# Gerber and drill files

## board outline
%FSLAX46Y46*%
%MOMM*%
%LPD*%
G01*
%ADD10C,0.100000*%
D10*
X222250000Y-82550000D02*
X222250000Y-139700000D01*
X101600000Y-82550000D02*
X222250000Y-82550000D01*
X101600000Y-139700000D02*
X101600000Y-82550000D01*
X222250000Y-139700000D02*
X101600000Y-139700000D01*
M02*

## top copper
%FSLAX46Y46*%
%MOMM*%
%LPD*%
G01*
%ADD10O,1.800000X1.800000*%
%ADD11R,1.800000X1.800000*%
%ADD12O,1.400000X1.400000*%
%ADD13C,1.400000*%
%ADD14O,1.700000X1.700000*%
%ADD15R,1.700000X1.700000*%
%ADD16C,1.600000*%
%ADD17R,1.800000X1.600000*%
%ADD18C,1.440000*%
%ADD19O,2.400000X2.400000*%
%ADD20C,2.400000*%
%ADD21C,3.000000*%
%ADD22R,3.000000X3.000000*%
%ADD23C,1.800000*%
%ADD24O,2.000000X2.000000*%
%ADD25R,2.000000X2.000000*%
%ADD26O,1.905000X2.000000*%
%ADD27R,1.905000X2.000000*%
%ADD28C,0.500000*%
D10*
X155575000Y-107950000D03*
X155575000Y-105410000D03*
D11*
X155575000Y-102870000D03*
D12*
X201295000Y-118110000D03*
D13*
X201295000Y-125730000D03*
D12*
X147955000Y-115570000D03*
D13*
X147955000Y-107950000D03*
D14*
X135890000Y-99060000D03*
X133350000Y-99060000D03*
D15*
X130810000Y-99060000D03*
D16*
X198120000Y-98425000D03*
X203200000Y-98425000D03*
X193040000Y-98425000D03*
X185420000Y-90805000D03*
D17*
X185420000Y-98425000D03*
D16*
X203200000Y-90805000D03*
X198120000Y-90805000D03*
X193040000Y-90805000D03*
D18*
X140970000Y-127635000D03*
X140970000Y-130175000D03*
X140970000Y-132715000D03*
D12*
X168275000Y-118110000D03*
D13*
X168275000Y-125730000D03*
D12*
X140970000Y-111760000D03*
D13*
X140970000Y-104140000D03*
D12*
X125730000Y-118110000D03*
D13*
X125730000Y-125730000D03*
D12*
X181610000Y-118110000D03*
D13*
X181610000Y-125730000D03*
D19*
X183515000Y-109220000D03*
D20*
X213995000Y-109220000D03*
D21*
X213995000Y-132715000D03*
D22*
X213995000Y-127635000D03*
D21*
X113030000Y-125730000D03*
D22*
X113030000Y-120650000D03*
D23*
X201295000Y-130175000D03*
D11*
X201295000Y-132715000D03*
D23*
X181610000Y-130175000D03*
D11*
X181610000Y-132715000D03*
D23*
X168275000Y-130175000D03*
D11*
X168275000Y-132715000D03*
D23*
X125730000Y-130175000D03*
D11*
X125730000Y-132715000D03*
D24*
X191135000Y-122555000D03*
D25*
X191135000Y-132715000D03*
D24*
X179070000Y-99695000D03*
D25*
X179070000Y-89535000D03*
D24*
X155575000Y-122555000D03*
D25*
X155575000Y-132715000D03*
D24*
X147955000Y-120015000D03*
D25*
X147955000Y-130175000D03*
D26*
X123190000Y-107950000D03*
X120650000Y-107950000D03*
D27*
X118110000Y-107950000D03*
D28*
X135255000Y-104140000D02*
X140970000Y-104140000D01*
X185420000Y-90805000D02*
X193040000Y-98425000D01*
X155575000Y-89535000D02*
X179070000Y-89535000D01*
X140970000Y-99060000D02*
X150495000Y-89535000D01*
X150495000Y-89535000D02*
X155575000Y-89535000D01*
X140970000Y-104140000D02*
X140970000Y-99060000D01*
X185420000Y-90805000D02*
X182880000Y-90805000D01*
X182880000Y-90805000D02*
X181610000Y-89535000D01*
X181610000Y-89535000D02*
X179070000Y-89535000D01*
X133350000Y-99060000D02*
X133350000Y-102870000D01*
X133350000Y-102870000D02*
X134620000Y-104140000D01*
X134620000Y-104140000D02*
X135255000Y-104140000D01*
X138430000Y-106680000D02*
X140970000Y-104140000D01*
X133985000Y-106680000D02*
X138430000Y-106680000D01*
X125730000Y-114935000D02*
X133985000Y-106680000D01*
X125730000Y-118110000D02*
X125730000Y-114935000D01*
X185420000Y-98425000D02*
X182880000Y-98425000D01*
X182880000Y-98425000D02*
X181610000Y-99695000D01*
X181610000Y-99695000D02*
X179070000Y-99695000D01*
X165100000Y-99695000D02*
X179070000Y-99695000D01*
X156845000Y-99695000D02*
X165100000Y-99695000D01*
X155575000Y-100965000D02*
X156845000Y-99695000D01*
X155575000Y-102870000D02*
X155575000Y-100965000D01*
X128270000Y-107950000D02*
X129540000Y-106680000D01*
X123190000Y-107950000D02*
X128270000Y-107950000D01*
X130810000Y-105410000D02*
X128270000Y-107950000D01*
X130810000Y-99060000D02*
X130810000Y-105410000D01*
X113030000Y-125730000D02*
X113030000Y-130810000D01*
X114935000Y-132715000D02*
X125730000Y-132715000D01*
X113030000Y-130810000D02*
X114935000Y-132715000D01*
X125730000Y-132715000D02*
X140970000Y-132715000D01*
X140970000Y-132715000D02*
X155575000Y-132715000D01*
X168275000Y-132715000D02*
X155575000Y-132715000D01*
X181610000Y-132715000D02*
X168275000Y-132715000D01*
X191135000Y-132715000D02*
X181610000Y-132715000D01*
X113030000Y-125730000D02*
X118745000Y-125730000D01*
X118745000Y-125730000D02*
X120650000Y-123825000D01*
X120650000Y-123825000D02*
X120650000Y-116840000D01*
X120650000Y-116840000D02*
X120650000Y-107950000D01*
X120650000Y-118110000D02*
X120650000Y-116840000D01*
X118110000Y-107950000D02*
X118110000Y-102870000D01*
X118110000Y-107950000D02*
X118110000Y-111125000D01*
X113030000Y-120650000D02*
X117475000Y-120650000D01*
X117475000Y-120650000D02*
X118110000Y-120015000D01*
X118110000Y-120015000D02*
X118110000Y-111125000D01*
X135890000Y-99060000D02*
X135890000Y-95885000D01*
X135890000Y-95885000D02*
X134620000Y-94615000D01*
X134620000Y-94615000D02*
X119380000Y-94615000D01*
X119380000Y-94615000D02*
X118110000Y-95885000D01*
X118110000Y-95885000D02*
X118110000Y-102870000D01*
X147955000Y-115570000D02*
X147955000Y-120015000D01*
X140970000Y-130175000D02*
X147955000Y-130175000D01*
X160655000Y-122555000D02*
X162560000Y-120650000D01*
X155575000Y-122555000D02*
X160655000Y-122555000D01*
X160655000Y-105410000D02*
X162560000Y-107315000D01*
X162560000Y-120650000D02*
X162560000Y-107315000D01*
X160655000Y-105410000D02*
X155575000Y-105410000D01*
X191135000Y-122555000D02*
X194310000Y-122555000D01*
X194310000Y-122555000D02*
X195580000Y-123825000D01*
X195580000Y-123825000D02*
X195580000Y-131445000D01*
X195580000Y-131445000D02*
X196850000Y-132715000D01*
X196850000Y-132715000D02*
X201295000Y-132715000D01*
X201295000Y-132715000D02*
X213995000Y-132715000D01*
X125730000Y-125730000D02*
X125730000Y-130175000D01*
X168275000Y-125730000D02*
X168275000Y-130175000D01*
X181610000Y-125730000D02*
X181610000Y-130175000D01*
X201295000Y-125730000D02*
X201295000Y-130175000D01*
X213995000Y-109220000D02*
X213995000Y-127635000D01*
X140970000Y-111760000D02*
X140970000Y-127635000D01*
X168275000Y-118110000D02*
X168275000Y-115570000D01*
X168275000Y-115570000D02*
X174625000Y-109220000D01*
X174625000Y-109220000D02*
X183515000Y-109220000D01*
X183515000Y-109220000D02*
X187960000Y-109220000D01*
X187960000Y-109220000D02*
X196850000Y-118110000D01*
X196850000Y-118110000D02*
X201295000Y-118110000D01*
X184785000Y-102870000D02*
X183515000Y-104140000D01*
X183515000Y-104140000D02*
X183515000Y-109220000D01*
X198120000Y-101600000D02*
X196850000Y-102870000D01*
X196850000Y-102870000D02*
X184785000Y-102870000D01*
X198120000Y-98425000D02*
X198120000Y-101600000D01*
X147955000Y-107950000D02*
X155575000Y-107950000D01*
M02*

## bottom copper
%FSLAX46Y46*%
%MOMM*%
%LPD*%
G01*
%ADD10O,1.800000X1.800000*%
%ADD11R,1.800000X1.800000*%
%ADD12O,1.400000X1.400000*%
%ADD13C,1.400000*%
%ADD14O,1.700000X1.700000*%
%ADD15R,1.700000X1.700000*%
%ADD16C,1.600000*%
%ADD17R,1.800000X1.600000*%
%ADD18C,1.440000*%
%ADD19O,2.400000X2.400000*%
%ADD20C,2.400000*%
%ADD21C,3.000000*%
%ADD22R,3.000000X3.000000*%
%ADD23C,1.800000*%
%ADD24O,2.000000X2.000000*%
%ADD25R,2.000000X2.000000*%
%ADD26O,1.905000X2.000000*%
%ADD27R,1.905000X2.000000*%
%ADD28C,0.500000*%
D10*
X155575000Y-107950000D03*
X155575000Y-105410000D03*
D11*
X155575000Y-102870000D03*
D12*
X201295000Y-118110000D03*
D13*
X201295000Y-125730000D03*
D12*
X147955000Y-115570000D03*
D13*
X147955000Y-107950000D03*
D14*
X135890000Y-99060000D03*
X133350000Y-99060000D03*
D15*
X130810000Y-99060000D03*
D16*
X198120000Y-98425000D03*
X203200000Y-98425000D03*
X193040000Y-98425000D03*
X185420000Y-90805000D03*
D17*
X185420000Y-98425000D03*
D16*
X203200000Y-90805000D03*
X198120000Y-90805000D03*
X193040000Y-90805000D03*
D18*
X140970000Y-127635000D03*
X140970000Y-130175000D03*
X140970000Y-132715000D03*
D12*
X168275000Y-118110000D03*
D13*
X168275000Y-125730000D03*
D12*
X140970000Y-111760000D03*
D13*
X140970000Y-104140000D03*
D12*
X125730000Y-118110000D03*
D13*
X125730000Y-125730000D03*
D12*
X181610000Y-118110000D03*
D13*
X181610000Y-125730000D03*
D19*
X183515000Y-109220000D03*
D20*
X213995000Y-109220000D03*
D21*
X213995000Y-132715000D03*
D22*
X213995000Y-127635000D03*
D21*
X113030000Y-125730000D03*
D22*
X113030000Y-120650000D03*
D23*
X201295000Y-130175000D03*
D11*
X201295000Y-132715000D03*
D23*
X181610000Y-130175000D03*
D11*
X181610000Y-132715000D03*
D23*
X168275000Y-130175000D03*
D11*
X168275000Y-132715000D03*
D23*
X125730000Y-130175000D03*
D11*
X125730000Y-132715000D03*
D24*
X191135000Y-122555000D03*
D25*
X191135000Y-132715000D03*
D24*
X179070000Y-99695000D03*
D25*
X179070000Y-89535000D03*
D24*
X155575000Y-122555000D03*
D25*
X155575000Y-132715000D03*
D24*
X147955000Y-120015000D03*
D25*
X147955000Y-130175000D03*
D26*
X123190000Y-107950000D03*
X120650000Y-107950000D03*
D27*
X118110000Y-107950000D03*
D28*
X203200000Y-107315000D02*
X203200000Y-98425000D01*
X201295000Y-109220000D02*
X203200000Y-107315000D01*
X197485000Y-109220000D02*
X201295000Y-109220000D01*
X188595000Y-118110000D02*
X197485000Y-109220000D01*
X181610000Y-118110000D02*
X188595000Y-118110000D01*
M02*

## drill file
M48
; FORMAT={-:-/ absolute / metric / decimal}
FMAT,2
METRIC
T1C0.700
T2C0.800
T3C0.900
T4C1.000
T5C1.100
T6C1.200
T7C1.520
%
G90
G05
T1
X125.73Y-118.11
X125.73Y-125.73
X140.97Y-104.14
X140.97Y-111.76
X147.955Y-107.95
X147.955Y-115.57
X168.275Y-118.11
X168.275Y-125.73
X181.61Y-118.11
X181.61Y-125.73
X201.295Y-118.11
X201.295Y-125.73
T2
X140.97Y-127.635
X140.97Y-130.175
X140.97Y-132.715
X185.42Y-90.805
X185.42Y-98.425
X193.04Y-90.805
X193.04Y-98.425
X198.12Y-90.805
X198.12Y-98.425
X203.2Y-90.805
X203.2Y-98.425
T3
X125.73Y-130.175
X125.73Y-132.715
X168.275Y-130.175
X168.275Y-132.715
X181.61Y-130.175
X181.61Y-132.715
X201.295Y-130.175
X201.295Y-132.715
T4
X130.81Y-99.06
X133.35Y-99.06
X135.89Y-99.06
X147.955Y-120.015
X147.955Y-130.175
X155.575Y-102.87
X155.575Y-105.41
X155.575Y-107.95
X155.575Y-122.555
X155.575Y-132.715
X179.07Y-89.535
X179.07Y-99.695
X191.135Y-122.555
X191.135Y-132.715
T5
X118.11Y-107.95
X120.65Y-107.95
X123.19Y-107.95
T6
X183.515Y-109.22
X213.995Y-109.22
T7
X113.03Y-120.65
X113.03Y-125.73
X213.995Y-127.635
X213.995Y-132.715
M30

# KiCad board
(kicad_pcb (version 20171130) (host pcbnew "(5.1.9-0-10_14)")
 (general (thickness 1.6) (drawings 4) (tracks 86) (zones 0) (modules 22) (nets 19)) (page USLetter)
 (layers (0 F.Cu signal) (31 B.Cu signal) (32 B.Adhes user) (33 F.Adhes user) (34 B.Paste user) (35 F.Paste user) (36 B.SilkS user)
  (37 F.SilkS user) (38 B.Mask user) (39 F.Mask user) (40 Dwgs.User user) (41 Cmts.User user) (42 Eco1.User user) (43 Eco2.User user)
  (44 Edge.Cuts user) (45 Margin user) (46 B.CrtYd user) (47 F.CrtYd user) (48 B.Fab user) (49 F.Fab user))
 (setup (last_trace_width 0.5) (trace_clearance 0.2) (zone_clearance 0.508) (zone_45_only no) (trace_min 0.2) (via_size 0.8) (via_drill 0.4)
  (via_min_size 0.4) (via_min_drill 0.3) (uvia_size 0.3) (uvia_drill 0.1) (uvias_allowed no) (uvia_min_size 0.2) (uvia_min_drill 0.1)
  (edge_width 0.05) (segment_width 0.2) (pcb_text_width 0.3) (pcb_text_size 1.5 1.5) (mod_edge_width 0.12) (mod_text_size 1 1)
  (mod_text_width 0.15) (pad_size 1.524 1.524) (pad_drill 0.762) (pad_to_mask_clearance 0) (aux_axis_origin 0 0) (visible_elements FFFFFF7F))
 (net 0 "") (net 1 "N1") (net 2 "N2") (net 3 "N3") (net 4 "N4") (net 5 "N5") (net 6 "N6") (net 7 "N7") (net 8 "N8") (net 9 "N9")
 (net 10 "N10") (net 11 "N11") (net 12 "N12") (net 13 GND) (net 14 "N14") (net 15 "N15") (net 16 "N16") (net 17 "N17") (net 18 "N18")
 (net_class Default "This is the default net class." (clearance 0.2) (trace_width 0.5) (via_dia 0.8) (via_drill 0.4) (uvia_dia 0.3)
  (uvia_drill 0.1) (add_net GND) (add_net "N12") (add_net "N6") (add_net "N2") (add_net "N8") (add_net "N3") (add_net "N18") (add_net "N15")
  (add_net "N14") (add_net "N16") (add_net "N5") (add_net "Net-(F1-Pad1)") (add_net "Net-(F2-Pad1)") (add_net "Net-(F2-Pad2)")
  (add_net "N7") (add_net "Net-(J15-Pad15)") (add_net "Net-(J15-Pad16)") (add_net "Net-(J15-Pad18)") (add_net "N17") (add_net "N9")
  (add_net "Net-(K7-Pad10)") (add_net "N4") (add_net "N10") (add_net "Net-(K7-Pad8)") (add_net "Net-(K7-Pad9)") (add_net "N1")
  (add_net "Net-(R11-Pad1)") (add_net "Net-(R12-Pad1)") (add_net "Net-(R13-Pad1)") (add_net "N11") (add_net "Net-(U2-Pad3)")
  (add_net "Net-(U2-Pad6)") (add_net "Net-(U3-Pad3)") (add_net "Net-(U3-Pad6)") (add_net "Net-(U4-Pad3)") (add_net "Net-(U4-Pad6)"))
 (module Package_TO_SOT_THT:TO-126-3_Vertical (layer F.Cu) (at 155.575 102.87 270)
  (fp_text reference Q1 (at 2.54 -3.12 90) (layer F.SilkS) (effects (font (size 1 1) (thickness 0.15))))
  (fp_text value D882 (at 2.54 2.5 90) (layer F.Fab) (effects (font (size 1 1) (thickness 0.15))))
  (pad 3 thru_hole oval (at 5.08 0 270) (size 1.8 1.8) (drill 1) (layers *.Cu *.Mask) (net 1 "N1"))
  (pad 2 thru_hole oval (at 2.54 0 270) (size 1.8 1.8) (drill 1) (layers *.Cu *.Mask) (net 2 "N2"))
  (pad 1 thru_hole rect (at 0 0 270) (size 1.8 1.8) (drill 1) (layers *.Cu *.Mask) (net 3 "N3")))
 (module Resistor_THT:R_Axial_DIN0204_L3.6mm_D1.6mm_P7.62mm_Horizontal (layer F.Cu) (at 201.295 125.73 90)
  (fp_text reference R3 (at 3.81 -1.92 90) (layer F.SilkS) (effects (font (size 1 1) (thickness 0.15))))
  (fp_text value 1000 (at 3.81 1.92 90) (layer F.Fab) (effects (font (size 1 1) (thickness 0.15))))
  (pad 2 thru_hole oval (at 7.62 0 90) (size 1.4 1.4) (drill 0.7) (layers *.Cu *.Mask) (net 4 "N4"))
  (pad 1 thru_hole circle (at 0 0 90) (size 1.4 1.4) (drill 0.7) (layers *.Cu *.Mask) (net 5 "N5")))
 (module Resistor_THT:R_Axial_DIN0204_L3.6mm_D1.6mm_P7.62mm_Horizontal (layer F.Cu) (at 147.955 107.95 270)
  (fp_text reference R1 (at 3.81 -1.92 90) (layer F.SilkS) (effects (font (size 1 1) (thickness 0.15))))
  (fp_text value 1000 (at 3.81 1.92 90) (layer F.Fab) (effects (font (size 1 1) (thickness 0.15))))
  (pad 2 thru_hole oval (at 7.62 0 270) (size 1.4 1.4) (drill 0.7) (layers *.Cu *.Mask) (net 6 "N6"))
  (pad 1 thru_hole circle (at 0 0 270) (size 1.4 1.4) (drill 0.7) (layers *.Cu *.Mask) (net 1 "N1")))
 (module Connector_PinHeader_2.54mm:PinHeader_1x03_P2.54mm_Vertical (layer F.Cu) (at 130.81 99.06 90)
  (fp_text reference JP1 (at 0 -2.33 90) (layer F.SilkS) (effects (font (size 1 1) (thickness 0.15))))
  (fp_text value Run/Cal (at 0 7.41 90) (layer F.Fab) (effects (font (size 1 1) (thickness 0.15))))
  (pad 3 thru_hole oval (at 0 5.08 90) (size 1.7 1.7) (drill 1) (layers *.Cu *.Mask) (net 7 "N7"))
  (pad 2 thru_hole oval (at 0 2.54 90) (size 1.7 1.7) (drill 1) (layers *.Cu *.Mask) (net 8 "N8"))
  (pad 1 thru_hole rect (at 0 0 90) (size 1.7 1.7) (drill 1) (layers *.Cu *.Mask) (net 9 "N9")))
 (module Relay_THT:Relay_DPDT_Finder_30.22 (layer F.Cu) (at 185.42 98.425)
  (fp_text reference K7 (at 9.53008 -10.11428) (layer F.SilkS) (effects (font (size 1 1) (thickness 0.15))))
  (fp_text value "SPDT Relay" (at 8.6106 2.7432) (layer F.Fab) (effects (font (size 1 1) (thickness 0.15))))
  (pad 3 thru_hole circle (at 12.7 0 90) (size 1.6 1.6) (drill 0.8) (layers *.Cu *.Mask) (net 4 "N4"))
  (pad 5 thru_hole circle (at 17.78 0 90) (size 1.6 1.6) (drill 0.8) (layers *.Cu *.Mask) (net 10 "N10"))
  (pad 4 thru_hole circle (at 7.62 0 90) (size 1.6 1.6) (drill 0.8) (layers *.Cu *.Mask) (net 8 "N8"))
  (pad 12 thru_hole circle (at 0 -7.62 90) (size 1.6 1.6) (drill 0.8) (layers *.Cu *.Mask) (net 8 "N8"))
  (pad 1 thru_hole rect (at 0 0 90) (size 1.6 1.8) (drill 0.8) (layers *.Cu *.Mask) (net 3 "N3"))
  (pad 8 thru_hole circle (at 17.78 -7.62 180) (size 1.6 1.6) (drill 0.8) (layers *.Cu *.Mask))
  (pad 10 thru_hole circle (at 12.7 -7.62 90) (size 1.6 1.6) (drill 0.8) (layers *.Cu *.Mask))
  (pad 9 thru_hole circle (at 7.62 -7.62 90) (size 1.6 1.6) (drill 0.8) (layers *.Cu *.Mask)))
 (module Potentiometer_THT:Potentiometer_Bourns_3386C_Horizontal (layer F.Cu) (at 140.97 127.635)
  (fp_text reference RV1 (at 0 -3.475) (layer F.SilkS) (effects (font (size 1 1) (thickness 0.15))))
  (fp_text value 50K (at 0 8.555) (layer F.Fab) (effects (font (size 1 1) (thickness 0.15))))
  (pad 1 thru_hole circle (at 0 0) (size 1.44 1.44) (drill 0.8) (layers *.Cu *.Mask) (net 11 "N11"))
  (pad 2 thru_hole circle (at 0 2.54) (size 1.44 1.44) (drill 0.8) (layers *.Cu *.Mask) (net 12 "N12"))
  (pad 3 thru_hole circle (at 0 5.08) (size 1.44 1.44) (drill 0.8) (layers *.Cu *.Mask) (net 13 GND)))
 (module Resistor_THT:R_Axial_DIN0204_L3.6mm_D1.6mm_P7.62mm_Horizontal (layer F.Cu) (at 168.275 125.73 90)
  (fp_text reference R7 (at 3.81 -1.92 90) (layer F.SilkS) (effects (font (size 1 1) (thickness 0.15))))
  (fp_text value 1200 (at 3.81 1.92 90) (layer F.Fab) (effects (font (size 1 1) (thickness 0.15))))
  (pad 2 thru_hole oval (at 7.62 0 90) (size 1.4 1.4) (drill 0.7) (layers *.Cu *.Mask) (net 4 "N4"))
  (pad 1 thru_hole circle (at 0 0 90) (size 1.4 1.4) (drill 0.7) (layers *.Cu *.Mask) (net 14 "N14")))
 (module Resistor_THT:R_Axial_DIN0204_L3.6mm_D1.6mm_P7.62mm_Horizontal (layer F.Cu) (at 140.97 104.14 270)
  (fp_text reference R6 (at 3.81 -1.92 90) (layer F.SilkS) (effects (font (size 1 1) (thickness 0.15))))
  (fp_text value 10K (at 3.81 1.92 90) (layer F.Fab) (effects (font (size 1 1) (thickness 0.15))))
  (pad 2 thru_hole oval (at 7.62 0 270) (size 1.4 1.4) (drill 0.7) (layers *.Cu *.Mask) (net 11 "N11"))
  (pad 1 thru_hole circle (at 0 0 270) (size 1.4 1.4) (drill 0.7) (layers *.Cu *.Mask) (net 8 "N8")))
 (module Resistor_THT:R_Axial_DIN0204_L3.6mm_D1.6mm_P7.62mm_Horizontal (layer F.Cu) (at 125.73 125.73 90)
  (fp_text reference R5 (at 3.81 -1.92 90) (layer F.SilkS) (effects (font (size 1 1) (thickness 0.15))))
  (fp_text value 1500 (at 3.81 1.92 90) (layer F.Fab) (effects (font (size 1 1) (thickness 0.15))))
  (pad 2 thru_hole oval (at 7.62 0 90) (size 1.4 1.4) (drill 0.7) (layers *.Cu *.Mask) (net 8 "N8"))
  (pad 1 thru_hole circle (at 0 0 90) (size 1.4 1.4) (drill 0.7) (layers *.Cu *.Mask) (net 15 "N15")))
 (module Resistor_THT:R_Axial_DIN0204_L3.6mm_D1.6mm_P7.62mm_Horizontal (layer F.Cu) (at 181.61 125.73 90)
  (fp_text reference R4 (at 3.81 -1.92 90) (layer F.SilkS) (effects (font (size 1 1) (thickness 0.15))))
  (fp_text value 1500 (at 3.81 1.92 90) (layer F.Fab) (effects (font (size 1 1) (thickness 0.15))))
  (pad 2 thru_hole oval (at 7.62 0 90) (size 1.4 1.4) (drill 0.7) (layers *.Cu *.Mask) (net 10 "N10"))
  (pad 1 thru_hole circle (at 0 0 90) (size 1.4 1.4) (drill 0.7) (layers *.Cu *.Mask) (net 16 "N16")))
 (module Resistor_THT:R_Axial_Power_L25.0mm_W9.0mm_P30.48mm (layer F.Cu) (at 213.995 109.22 180)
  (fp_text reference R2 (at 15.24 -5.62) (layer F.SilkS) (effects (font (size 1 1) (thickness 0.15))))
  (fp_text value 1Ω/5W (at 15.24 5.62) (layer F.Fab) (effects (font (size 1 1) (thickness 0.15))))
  (pad 2 thru_hole oval (at 30.48 0 180) (size 2.4 2.4) (drill 1.2) (layers *.Cu *.Mask) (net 4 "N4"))
  (pad 1 thru_hole circle (at 0 0 180) (size 2.4 2.4) (drill 1.2) (layers *.Cu *.Mask) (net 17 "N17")))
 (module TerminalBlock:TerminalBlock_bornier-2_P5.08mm (layer F.Cu) (at 213.995 127.635 270)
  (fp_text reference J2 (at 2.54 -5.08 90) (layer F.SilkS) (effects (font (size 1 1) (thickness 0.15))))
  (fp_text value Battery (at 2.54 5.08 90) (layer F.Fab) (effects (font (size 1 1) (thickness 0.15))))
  (pad 2 thru_hole circle (at 5.08 0 270) (size 3 3) (drill 1.52) (layers *.Cu *.Mask) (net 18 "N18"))
  (pad 1 thru_hole rect (at 0 0 270) (size 3 3) (drill 1.52) (layers *.Cu *.Mask) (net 17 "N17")))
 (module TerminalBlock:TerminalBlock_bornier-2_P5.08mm (layer F.Cu) (at 113.03 120.65 270)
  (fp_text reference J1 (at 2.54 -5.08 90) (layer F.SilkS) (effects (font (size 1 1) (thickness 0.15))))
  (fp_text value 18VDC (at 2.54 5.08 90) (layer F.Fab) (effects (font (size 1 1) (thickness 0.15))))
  (pad 2 thru_hole circle (at 5.08 0 270) (size 3 3) (drill 1.52) (layers *.Cu *.Mask) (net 13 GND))
  (pad 1 thru_hole rect (at 0 0 270) (size 3 3) (drill 1.52) (layers *.Cu *.Mask) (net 7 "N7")))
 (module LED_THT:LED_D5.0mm (layer F.Cu) (at 201.295 132.715 90)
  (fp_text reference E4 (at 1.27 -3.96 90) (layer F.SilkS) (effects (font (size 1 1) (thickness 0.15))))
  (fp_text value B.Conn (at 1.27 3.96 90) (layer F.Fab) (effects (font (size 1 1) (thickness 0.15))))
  (pad 2 thru_hole circle (at 2.54 0 90) (size 1.8 1.8) (drill 0.9) (layers *.Cu *.Mask) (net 5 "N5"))
  (pad 1 thru_hole rect (at 0 0 90) (size 1.8 1.8) (drill 0.9) (layers *.Cu *.Mask) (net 18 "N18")))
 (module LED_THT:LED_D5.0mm (layer F.Cu) (at 181.61 132.715 90)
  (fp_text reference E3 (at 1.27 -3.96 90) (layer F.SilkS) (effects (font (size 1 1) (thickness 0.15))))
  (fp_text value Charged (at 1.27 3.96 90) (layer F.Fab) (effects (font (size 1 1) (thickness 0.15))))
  (pad 2 thru_hole circle (at 2.54 0 90) (size 1.8 1.8) (drill 0.9) (layers *.Cu *.Mask) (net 16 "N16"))
  (pad 1 thru_hole rect (at 0 0 90) (size 1.8 1.8) (drill 0.9) (layers *.Cu *.Mask) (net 13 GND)))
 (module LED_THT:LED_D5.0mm (layer F.Cu) (at 168.275 132.715 90)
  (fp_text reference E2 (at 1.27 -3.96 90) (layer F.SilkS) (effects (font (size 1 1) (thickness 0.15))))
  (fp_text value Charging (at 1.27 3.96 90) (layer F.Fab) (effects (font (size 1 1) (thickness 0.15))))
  (pad 2 thru_hole circle (at 2.54 0 90) (size 1.8 1.8) (drill 0.9) (layers *.Cu *.Mask) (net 14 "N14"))
  (pad 1 thru_hole rect (at 0 0 90) (size 1.8 1.8) (drill 0.9) (layers *.Cu *.Mask) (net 13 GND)))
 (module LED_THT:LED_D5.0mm (layer F.Cu) (at 125.73 132.715 90)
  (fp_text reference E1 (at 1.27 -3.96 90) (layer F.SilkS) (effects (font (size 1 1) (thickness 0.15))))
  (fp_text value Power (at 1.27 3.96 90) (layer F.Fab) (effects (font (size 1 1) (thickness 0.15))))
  (pad 2 thru_hole circle (at 2.54 0 90) (size 1.8 1.8) (drill 0.9) (layers *.Cu *.Mask) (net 15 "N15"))
  (pad 1 thru_hole rect (at 0 0 90) (size 1.8 1.8) (drill 0.9) (layers *.Cu *.Mask) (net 13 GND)))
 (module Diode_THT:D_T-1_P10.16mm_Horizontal (layer F.Cu) (at 191.135 132.715 90)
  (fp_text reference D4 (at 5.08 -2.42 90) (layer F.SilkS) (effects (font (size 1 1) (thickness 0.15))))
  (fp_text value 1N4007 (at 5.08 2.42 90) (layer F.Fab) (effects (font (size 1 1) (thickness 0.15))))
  (pad 2 thru_hole oval (at 10.16 0 90) (size 2 2) (drill 1) (layers *.Cu *.Mask) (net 18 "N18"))
  (pad 1 thru_hole rect (at 0 0 90) (size 2 2) (drill 1) (layers *.Cu *.Mask) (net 13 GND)))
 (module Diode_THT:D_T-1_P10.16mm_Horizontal (layer F.Cu) (at 179.07 89.535 270)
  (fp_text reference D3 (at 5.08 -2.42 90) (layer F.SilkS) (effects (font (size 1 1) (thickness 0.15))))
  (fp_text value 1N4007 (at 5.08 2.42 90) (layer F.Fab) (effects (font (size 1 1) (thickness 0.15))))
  (pad 2 thru_hole oval (at 10.16 0 270) (size 2 2) (drill 1) (layers *.Cu *.Mask) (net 3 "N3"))
  (pad 1 thru_hole rect (at 0 0 270) (size 2 2) (drill 1) (layers *.Cu *.Mask) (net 8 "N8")))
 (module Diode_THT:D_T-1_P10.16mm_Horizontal (layer F.Cu) (at 155.575 132.715 90)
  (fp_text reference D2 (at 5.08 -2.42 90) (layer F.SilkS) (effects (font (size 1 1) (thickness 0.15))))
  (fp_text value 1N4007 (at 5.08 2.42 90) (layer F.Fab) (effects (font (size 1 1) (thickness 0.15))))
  (pad 2 thru_hole oval (at 10.16 0 90) (size 2 2) (drill 1) (layers *.Cu *.Mask) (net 2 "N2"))
  (pad 1 thru_hole rect (at 0 0 90) (size 2 2) (drill 1) (layers *.Cu *.Mask) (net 13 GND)))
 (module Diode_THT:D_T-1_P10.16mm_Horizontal (layer F.Cu) (at 147.955 130.175 90)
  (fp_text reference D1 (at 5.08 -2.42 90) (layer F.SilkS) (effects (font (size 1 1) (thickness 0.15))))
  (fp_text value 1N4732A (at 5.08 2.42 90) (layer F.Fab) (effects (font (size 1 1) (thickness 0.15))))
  (pad 2 thru_hole oval (at 10.16 0 90) (size 2 2) (drill 1) (layers *.Cu *.Mask) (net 6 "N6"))
  (pad 1 thru_hole rect (at 0 0 90) (size 2 2) (drill 1) (layers *.Cu *.Mask) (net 12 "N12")))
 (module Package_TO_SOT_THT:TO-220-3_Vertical (layer F.Cu) (at 118.11 107.95)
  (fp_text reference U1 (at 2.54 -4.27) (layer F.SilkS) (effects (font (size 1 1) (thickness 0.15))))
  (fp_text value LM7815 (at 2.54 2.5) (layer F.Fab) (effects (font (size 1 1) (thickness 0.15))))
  (pad 3 thru_hole oval (at 5.08 0) (size 1.905 2) (drill 1.1) (layers *.Cu *.Mask) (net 9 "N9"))
  (pad 2 thru_hole oval (at 2.54 0) (size 1.905 2) (drill 1.1) (layers *.Cu *.Mask) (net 13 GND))
  (pad 1 thru_hole rect (at 0 0) (size 1.905 2) (drill 1.1) (layers *.Cu *.Mask) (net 7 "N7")))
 (gr_line (start 222.25 82.55) (end 222.25 139.7) (layer Edge.Cuts) (width 0.1))
 (gr_line (start 101.6 82.55) (end 222.25 82.55) (layer Edge.Cuts) (width 0.1))
 (gr_line (start 101.6 139.7) (end 101.6 82.55) (layer Edge.Cuts) (width 0.1))
 (gr_line (start 222.25 139.7) (end 101.6 139.7) (layer Edge.Cuts) (width 0.1))
 (segment (start 135.255 104.14) (end 140.97 104.14) (width 0.5) (layer F.Cu) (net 8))
 (segment (start 185.42 90.805) (end 193.04 98.425) (width 0.5) (layer F.Cu) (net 8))
 (segment (start 155.575 89.535) (end 179.07 89.535) (width 0.5) (layer F.Cu) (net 8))
 (segment (start 140.97 99.06) (end 150.495 89.535) (width 0.5) (layer F.Cu) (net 8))
 (segment (start 150.495 89.535) (end 155.575 89.535) (width 0.5) (layer F.Cu) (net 8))
 (segment (start 140.97 104.14) (end 140.97 99.06) (width 0.5) (layer F.Cu) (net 8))
 (segment (start 185.42 90.805) (end 182.88 90.805) (width 0.5) (layer F.Cu) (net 8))
 (segment (start 182.88 90.805) (end 181.61 89.535) (width 0.5) (layer F.Cu) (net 8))
 (segment (start 181.61 89.535) (end 179.07 89.535) (width 0.5) (layer F.Cu) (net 8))
 (segment (start 133.35 99.06) (end 133.35 102.87) (width 0.5) (layer F.Cu) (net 8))
 (segment (start 133.35 102.87) (end 134.62 104.14) (width 0.5) (layer F.Cu) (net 8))
 (segment (start 134.62 104.14) (end 135.255 104.14) (width 0.5) (layer F.Cu) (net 8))
 (segment (start 138.43 106.68) (end 140.97 104.14) (width 0.5) (layer F.Cu) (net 8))
 (segment (start 133.985 106.68) (end 138.43 106.68) (width 0.5) (layer F.Cu) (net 8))
 (segment (start 125.73 114.935) (end 133.985 106.68) (width 0.5) (layer F.Cu) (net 8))
 (segment (start 125.73 118.11) (end 125.73 114.935) (width 0.5) (layer F.Cu) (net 8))
 (segment (start 185.42 98.425) (end 182.88 98.425) (width 0.5) (layer F.Cu) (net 3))
 (segment (start 182.88 98.425) (end 181.61 99.695) (width 0.5) (layer F.Cu) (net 3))
 (segment (start 181.61 99.695) (end 179.07 99.695) (width 0.5) (layer F.Cu) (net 3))
 (segment (start 165.1 99.695) (end 179.07 99.695) (width 0.5) (layer F.Cu) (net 3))
 (segment (start 156.845 99.695) (end 165.1 99.695) (width 0.5) (layer F.Cu) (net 3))
 (segment (start 155.575 100.965) (end 156.845 99.695) (width 0.5) (layer F.Cu) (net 3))
 (segment (start 155.575 102.87) (end 155.575 100.965) (width 0.5) (layer F.Cu) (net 3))
 (segment (start 128.27 107.95) (end 129.54 106.68) (width 0.5) (layer F.Cu) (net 9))
 (segment (start 123.19 107.95) (end 128.27 107.95) (width 0.5) (layer F.Cu) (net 9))
 (segment (start 130.81 105.41) (end 128.27 107.95) (width 0.5) (layer F.Cu) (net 9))
 (segment (start 130.81 99.06) (end 130.81 105.41) (width 0.5) (layer F.Cu) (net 9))
 (segment (start 113.03 125.73) (end 113.03 130.81) (width 0.5) (layer F.Cu) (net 13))
 (segment (start 114.935 132.715) (end 125.73 132.715) (width 0.5) (layer F.Cu) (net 13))
 (segment (start 113.03 130.81) (end 114.935 132.715) (width 0.5) (layer F.Cu) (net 13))
 (segment (start 125.73 132.715) (end 140.97 132.715) (width 0.5) (layer F.Cu) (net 13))
 (segment (start 140.97 132.715) (end 155.575 132.715) (width 0.5) (layer F.Cu) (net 13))
 (segment (start 168.275 132.715) (end 155.575 132.715) (width 0.5) (layer F.Cu) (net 13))
 (segment (start 181.61 132.715) (end 168.275 132.715) (width 0.5) (layer F.Cu) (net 13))
 (segment (start 191.135 132.715) (end 181.61 132.715) (width 0.5) (layer F.Cu) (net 13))
 (segment (start 113.03 125.73) (end 118.745 125.73) (width 0.5) (layer F.Cu) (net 13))
 (segment (start 118.745 125.73) (end 120.65 123.825) (width 0.5) (layer F.Cu) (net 13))
 (segment (start 120.65 123.825) (end 120.65 116.84) (width 0.5) (layer F.Cu) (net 13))
 (segment (start 120.65 116.84) (end 120.65 107.95) (width 0.5) (layer F.Cu) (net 13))
 (segment (start 120.65 118.11) (end 120.65 116.84) (width 0.5) (layer F.Cu) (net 13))
 (segment (start 118.11 107.95) (end 118.11 102.87) (width 0.5) (layer F.Cu) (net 7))
 (segment (start 118.11 107.95) (end 118.11 111.125) (width 0.5) (layer F.Cu) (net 7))
 (segment (start 113.03 120.65) (end 117.475 120.65) (width 0.5) (layer F.Cu) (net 7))
 (segment (start 117.475 120.65) (end 118.11 120.015) (width 0.5) (layer F.Cu) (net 7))
 (segment (start 118.11 120.015) (end 118.11 111.125) (width 0.5) (layer F.Cu) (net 7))
 (segment (start 135.89 99.06) (end 135.89 95.885) (width 0.5) (layer F.Cu) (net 7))
 (segment (start 135.89 95.885) (end 134.62 94.615) (width 0.5) (layer F.Cu) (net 7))
 (segment (start 134.62 94.615) (end 119.38 94.615) (width 0.5) (layer F.Cu) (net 7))
 (segment (start 119.38 94.615) (end 118.11 95.885) (width 0.5) (layer F.Cu) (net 7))
 (segment (start 118.11 95.885) (end 118.11 102.87) (width 0.5) (layer F.Cu) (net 7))
 (segment (start 147.955 115.57) (end 147.955 120.015) (width 0.5) (layer F.Cu) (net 6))
 (segment (start 140.97 130.175) (end 147.955 130.175) (width 0.5) (layer F.Cu) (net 12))
 (segment (start 160.655 122.555) (end 162.56 120.65) (width 0.5) (layer F.Cu) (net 2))
 (segment (start 155.575 122.555) (end 160.655 122.555) (width 0.5) (layer F.Cu) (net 2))
 (segment (start 160.655 105.41) (end 162.56 107.315) (width 0.5) (layer F.Cu) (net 2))
 (segment (start 162.56 120.65) (end 162.56 107.315) (width 0.5) (layer F.Cu) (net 2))
 (segment (start 160.655 105.41) (end 155.575 105.41) (width 0.5) (layer F.Cu) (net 2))
 (segment (start 191.135 122.555) (end 194.31 122.555) (width 0.5) (layer F.Cu) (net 18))
 (segment (start 194.31 122.555) (end 195.58 123.825) (width 0.5) (layer F.Cu) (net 18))
 (segment (start 195.58 123.825) (end 195.58 131.445) (width 0.5) (layer F.Cu) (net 18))
 (segment (start 195.58 131.445) (end 196.85 132.715) (width 0.5) (layer F.Cu) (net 18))
 (segment (start 196.85 132.715) (end 201.295 132.715) (width 0.5) (layer F.Cu) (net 18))
 (segment (start 201.295 132.715) (end 213.995 132.715) (width 0.5) (layer F.Cu) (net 18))
 (segment (start 125.73 125.73) (end 125.73 130.175) (width 0.5) (layer F.Cu) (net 15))
 (segment (start 168.275 125.73) (end 168.275 130.175) (width 0.5) (layer F.Cu) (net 14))
 (segment (start 181.61 125.73) (end 181.61 130.175) (width 0.5) (layer F.Cu) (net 16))
 (segment (start 201.295 125.73) (end 201.295 130.175) (width 0.5) (layer F.Cu) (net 5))
 (segment (start 213.995 109.22) (end 213.995 127.635) (width 0.5) (layer F.Cu) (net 17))
 (segment (start 140.97 111.76) (end 140.97 127.635) (width 0.5) (layer F.Cu) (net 11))
 (segment (start 168.275 118.11) (end 168.275 115.57) (width 0.5) (layer F.Cu) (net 4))
 (segment (start 168.275 115.57) (end 174.625 109.22) (width 0.5) (layer F.Cu) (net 4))
 (segment (start 174.625 109.22) (end 183.515 109.22) (width 0.5) (layer F.Cu) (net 4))
 (segment (start 183.515 109.22) (end 187.96 109.22) (width 0.5) (layer F.Cu) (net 4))
 (segment (start 187.96 109.22) (end 196.85 118.11) (width 0.5) (layer F.Cu) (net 4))
 (segment (start 196.85 118.11) (end 201.295 118.11) (width 0.5) (layer F.Cu) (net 4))
 (segment (start 184.785 102.87) (end 183.515 104.14) (width 0.5) (layer F.Cu) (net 4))
 (segment (start 183.515 104.14) (end 183.515 109.22) (width 0.5) (layer F.Cu) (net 4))
 (segment (start 198.12 101.6) (end 196.85 102.87) (width 0.5) (layer F.Cu) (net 4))
 (segment (start 196.85 102.87) (end 184.785 102.87) (width 0.5) (layer F.Cu) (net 4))
 (segment (start 198.12 98.425) (end 198.12 101.6) (width 0.5) (layer F.Cu) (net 4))
 (segment (start 203.2 107.315) (end 203.2 98.425) (width 0.5) (layer B.Cu) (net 10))
 (segment (start 201.295 109.22) (end 203.2 107.315) (width 0.5) (layer B.Cu) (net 10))
 (segment (start 197.485 109.22) (end 201.295 109.22) (width 0.5) (layer B.Cu) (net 10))
 (segment (start 188.595 118.11) (end 197.485 109.22) (width 0.5) (layer B.Cu) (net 10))
 (segment (start 181.61 118.11) (end 188.595 118.11) (width 0.5) (layer B.Cu) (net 10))
 (segment (start 147.955 107.95) (end 155.575 107.95) (width 0.5) (layer F.Cu) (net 1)))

